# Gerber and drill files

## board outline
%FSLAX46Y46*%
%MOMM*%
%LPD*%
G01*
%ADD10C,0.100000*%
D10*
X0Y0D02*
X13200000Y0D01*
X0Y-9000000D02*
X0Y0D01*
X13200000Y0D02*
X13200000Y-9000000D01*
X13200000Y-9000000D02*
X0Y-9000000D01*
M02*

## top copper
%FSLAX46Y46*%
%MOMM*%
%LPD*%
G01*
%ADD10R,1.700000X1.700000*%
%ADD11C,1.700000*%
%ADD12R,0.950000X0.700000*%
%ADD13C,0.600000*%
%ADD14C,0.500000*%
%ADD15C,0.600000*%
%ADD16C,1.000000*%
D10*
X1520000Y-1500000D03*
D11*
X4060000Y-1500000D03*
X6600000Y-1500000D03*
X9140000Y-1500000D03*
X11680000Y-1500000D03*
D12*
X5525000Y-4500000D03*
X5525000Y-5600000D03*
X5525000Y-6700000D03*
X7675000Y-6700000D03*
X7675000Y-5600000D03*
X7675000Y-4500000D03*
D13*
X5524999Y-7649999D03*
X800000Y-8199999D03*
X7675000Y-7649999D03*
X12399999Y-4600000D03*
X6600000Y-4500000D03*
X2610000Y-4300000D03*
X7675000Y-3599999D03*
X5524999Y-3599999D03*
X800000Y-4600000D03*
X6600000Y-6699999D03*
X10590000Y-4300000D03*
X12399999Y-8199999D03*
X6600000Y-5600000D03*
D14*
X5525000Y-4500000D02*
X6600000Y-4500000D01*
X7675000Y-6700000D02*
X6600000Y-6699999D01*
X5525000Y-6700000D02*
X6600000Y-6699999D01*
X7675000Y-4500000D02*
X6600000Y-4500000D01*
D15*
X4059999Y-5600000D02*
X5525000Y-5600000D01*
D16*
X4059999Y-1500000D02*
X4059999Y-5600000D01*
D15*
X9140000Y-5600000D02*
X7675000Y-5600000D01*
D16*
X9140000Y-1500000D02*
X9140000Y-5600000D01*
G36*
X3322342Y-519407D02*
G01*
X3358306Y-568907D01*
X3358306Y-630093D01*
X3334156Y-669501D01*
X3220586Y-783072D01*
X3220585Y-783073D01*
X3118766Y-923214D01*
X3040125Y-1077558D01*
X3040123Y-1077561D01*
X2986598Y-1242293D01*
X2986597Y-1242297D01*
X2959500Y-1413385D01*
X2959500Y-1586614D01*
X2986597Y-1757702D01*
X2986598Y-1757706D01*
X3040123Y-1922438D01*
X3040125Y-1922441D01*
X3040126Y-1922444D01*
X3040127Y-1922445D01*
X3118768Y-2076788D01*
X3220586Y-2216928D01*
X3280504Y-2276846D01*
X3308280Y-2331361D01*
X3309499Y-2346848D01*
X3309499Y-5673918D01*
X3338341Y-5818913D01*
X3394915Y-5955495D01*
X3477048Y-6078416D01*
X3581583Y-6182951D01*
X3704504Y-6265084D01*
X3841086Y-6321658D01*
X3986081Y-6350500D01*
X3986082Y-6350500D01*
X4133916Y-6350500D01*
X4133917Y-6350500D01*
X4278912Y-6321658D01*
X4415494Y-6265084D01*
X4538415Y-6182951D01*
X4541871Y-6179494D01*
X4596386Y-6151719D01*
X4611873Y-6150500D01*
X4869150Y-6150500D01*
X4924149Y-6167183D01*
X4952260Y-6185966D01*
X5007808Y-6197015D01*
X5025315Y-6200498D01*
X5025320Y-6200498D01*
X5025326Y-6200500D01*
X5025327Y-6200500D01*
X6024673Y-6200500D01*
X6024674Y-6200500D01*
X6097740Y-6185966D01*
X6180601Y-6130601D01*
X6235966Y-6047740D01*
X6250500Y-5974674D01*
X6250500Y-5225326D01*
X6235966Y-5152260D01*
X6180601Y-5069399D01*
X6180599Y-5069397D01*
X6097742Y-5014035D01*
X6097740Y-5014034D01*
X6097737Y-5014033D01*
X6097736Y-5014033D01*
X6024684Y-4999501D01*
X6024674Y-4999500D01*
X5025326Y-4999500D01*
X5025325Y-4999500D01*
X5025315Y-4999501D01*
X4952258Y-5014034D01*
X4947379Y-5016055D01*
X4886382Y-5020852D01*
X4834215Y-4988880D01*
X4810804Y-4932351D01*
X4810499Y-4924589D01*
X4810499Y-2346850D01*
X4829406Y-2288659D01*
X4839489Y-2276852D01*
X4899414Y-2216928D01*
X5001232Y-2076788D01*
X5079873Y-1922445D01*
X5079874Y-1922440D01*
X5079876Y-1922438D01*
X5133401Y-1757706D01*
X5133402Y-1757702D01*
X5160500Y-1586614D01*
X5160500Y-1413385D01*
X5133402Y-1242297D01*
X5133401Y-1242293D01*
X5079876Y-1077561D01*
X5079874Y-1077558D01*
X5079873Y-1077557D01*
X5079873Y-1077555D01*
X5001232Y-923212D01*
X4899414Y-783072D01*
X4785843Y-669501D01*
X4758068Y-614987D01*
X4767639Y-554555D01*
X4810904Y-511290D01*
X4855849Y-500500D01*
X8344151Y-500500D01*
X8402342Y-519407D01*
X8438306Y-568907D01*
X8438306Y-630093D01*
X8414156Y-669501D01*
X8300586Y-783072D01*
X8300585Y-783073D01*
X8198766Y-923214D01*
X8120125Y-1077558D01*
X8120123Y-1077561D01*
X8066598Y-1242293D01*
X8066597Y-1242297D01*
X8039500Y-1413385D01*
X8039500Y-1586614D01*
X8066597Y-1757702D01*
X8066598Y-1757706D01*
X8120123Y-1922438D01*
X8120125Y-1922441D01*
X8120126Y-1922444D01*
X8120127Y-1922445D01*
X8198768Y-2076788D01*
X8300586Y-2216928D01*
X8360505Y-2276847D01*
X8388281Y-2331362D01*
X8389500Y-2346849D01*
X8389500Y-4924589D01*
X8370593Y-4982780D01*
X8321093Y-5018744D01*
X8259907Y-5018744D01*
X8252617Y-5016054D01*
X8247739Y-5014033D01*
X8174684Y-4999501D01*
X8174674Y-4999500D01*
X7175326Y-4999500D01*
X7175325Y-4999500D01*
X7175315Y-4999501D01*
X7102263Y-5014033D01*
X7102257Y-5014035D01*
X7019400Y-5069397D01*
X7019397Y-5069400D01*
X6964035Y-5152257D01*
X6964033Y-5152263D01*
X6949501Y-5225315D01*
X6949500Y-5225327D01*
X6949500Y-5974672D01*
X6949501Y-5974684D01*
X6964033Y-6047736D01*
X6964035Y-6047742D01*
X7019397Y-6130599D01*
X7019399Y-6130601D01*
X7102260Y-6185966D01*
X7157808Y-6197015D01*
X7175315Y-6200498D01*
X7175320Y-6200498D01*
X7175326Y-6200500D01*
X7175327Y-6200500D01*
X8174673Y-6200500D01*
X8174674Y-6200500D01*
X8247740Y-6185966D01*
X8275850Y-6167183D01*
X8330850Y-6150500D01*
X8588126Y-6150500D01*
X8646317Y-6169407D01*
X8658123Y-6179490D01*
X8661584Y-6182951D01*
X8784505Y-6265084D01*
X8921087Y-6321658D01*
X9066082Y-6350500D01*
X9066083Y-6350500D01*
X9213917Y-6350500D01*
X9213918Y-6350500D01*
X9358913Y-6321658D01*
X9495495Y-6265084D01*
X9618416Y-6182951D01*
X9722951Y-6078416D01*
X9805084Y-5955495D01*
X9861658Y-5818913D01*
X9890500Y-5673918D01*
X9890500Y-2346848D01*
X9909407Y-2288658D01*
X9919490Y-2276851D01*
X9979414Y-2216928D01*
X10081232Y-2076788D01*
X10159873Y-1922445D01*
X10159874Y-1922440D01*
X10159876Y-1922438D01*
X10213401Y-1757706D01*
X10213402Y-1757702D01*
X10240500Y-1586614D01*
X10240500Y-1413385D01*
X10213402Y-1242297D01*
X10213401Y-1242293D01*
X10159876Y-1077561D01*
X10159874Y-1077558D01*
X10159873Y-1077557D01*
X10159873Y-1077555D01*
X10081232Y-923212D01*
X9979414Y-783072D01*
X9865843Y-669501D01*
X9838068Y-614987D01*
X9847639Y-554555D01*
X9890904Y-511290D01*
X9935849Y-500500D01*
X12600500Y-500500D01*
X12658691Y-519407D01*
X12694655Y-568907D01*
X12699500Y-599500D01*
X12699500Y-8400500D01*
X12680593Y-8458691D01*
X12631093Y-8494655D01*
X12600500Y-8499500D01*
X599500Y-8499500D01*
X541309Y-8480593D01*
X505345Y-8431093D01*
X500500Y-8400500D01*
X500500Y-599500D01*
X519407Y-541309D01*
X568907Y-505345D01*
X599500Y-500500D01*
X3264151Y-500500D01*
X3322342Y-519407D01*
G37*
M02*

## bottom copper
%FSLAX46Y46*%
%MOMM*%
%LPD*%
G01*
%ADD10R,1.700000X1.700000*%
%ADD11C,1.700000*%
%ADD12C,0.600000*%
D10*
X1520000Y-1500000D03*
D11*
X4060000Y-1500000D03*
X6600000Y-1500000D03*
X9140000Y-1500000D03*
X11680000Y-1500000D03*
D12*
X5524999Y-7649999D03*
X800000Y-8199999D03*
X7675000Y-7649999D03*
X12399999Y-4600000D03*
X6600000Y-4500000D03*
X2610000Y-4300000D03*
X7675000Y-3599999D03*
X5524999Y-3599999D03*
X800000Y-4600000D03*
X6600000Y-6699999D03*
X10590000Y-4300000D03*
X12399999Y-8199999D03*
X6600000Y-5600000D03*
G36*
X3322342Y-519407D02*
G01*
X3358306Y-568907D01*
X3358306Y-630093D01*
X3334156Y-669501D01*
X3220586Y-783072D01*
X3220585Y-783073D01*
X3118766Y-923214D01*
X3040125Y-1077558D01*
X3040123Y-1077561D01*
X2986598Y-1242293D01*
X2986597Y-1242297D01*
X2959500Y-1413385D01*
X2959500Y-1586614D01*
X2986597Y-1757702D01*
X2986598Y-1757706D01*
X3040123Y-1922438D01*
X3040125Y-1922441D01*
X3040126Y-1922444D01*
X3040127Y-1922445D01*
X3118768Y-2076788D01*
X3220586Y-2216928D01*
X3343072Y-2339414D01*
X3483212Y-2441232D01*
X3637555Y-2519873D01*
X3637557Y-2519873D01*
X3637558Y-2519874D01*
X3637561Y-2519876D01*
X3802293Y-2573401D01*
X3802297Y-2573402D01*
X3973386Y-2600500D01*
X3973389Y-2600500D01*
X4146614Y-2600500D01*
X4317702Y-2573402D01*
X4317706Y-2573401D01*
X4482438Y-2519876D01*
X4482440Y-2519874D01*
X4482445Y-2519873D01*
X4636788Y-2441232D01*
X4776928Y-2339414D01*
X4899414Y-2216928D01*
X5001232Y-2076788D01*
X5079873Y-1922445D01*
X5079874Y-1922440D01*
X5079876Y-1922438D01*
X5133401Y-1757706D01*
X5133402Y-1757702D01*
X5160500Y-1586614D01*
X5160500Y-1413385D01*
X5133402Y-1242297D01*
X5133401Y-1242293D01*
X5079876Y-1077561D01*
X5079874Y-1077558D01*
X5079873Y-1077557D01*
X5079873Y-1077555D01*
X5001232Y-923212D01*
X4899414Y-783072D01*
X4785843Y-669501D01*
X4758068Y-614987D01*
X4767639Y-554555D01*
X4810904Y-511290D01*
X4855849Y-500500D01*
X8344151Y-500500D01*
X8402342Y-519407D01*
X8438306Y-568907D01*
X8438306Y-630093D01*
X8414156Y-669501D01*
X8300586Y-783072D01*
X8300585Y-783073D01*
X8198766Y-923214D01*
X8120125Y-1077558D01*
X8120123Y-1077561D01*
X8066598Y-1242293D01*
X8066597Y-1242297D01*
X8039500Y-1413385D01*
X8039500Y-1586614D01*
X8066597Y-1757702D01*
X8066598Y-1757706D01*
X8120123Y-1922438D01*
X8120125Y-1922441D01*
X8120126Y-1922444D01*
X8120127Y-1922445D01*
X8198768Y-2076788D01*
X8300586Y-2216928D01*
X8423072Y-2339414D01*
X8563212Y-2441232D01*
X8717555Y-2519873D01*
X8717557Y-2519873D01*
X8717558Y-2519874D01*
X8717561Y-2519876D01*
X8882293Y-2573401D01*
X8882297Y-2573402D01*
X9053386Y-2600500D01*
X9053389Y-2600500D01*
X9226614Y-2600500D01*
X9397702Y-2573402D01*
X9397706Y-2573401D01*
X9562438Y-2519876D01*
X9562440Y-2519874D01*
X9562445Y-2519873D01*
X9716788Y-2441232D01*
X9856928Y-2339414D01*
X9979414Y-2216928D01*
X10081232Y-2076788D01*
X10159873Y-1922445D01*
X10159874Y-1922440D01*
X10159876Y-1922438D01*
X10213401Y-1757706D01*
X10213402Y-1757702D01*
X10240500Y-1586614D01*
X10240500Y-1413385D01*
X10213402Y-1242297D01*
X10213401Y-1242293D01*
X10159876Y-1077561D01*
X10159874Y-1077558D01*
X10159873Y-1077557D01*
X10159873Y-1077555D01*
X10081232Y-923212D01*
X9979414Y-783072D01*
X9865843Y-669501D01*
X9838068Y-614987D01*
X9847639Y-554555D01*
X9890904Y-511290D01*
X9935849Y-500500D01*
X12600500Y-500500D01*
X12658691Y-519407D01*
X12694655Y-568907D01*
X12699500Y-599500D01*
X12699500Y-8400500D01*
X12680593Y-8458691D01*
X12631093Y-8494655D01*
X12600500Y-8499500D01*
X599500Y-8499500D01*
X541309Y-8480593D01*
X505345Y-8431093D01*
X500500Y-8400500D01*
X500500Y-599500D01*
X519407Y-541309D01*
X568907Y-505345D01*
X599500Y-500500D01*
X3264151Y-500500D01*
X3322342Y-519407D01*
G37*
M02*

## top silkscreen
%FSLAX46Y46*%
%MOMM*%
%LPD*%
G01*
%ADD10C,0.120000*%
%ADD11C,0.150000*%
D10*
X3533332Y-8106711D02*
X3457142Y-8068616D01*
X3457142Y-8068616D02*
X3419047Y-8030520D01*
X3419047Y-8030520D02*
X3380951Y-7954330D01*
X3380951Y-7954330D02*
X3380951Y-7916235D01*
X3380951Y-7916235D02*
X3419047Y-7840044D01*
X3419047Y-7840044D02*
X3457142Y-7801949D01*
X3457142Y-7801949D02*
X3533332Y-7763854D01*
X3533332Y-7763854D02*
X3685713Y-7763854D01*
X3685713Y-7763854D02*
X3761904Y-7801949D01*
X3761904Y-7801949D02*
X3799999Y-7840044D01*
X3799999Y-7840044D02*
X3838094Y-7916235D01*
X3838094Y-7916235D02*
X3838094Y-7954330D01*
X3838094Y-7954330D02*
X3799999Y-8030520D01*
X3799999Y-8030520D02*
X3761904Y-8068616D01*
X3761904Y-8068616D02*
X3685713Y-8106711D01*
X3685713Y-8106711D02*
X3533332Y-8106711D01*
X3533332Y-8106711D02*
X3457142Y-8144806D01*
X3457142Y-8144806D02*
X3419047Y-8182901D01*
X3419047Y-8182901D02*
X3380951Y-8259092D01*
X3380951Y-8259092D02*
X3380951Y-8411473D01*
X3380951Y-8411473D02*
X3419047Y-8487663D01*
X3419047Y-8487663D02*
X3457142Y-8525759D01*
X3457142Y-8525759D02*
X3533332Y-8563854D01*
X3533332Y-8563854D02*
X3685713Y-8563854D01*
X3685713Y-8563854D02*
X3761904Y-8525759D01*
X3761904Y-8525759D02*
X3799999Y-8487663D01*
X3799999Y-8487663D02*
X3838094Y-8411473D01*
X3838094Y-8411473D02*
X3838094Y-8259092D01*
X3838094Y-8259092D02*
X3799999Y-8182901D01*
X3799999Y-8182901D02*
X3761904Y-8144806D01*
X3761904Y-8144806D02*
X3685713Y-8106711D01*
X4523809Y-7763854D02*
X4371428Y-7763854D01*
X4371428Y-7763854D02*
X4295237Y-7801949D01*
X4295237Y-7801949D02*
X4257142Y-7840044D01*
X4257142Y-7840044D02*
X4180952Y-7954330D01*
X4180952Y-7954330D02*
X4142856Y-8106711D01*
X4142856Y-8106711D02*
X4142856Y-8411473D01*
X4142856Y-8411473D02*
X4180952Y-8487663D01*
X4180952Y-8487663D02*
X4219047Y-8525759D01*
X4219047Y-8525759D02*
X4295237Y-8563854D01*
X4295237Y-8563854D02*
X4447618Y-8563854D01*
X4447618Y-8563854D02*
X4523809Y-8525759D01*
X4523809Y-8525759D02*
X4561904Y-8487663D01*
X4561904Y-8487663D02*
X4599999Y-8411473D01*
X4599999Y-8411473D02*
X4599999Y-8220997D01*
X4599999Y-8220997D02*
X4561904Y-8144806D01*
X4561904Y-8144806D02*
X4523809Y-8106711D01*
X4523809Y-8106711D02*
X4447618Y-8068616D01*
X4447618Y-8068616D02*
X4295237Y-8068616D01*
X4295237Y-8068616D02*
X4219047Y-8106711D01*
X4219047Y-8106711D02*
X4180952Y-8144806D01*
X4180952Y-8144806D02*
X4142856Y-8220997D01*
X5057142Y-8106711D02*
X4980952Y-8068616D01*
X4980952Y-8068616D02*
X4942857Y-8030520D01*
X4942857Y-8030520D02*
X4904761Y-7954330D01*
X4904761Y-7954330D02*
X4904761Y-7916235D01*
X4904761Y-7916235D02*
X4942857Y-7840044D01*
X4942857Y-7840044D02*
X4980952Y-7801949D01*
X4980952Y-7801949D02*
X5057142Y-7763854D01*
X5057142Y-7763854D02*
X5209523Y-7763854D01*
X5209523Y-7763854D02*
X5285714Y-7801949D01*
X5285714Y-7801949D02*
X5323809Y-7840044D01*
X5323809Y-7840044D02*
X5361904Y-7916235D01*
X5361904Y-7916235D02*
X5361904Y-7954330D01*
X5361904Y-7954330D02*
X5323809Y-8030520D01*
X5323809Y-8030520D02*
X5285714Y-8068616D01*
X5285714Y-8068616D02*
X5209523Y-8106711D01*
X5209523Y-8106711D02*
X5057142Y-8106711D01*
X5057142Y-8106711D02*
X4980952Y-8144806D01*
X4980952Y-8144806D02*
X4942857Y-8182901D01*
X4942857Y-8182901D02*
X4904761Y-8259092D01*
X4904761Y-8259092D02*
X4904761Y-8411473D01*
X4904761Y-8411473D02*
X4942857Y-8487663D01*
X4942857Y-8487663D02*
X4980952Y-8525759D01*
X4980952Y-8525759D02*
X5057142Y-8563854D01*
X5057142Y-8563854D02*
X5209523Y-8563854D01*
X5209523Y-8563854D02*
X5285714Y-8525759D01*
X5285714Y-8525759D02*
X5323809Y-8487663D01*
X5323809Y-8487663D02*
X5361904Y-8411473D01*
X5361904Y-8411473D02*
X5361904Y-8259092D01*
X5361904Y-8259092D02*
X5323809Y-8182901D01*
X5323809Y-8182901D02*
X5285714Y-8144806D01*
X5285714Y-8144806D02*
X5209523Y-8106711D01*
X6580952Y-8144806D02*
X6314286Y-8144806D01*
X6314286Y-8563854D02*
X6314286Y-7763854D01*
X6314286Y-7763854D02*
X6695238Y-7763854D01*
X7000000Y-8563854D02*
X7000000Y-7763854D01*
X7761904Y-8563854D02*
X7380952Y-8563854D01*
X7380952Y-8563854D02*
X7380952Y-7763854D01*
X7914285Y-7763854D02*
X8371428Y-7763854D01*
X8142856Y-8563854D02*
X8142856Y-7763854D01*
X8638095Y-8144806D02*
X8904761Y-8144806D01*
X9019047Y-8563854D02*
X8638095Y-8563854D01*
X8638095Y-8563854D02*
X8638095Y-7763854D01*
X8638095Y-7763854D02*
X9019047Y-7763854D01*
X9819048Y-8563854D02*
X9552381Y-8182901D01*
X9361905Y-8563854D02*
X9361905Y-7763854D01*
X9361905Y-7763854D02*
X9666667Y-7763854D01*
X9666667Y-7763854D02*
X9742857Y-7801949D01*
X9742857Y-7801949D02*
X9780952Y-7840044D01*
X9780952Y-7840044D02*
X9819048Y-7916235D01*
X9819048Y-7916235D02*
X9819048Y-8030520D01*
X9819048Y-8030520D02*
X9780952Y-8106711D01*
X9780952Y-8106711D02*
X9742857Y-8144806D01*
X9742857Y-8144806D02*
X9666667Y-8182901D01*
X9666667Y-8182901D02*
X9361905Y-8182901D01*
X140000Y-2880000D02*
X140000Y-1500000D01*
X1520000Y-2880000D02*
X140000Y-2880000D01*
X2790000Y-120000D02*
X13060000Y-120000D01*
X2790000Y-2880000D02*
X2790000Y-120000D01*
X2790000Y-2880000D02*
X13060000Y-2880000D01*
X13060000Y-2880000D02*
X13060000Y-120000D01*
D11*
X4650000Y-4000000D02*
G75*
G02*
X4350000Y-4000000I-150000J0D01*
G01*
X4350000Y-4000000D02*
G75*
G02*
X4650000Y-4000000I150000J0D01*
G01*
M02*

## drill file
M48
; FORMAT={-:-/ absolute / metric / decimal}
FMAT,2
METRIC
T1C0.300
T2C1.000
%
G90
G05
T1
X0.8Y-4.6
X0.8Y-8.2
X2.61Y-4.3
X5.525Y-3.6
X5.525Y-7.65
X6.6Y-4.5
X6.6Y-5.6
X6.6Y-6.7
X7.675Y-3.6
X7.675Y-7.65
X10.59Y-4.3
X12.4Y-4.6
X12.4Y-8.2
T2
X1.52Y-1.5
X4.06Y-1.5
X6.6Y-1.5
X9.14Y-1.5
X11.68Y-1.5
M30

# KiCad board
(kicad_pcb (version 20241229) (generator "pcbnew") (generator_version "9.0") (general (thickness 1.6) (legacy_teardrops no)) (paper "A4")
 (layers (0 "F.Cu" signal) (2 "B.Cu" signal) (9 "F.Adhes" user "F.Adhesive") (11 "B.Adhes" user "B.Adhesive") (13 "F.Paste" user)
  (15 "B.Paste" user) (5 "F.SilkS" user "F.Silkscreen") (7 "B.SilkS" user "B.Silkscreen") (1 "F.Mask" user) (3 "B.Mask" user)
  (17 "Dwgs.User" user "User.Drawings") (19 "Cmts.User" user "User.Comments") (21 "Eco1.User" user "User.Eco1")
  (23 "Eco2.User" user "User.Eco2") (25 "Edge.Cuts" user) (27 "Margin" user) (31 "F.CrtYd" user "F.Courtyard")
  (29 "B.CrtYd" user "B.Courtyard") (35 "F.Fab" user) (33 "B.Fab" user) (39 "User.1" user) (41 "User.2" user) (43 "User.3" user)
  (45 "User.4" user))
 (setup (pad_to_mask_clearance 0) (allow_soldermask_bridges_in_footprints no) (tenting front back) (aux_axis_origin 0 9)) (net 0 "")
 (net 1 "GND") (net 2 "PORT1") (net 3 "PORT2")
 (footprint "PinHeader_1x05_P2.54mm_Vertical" (layer "F.Cu") (at 1.52 1.5 90)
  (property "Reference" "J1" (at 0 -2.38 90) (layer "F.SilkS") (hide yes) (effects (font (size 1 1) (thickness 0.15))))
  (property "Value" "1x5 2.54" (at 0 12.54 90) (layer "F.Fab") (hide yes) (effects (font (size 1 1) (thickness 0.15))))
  (fp_line (start -1.38 -1.38) (end 0 -1.38) (stroke (width 0.12) (type solid)) (layer "F.SilkS"))
  (fp_line (start -1.38 0) (end -1.38 -1.38) (stroke (width 0.12) (type solid)) (layer "F.SilkS"))
  (fp_line (start 1.38 1.27) (end 1.38 11.54) (stroke (width 0.12) (type solid)) (layer "F.SilkS"))
  (fp_line (start -1.38 1.27) (end 1.38 1.27) (stroke (width 0.12) (type solid)) (layer "F.SilkS"))
  (fp_line (start -1.38 1.27) (end -1.38 11.54) (stroke (width 0.12) (type solid)) (layer "F.SilkS"))
  (fp_line (start -1.38 11.54) (end 1.38 11.54) (stroke (width 0.12) (type solid)) (layer "F.SilkS"))
  (pad "1" thru_hole rect (at 0 0 90) (size 1.7 1.7) (drill 1) (layers "*.Cu" "*.Mask") (remove_unused_layers no) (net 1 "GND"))
  (pad "2" thru_hole circle (at 0 2.54 90) (size 1.7 1.7) (drill 1) (layers "*.Cu" "*.Mask") (remove_unused_layers no) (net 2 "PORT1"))
  (pad "3" thru_hole circle (at 0 5.08 90) (size 1.7 1.7) (drill 1) (layers "*.Cu" "*.Mask") (remove_unused_layers no) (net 1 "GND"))
  (pad "4" thru_hole circle (at 0 7.62 90) (size 1.7 1.7) (drill 1) (layers "*.Cu" "*.Mask") (remove_unused_layers no) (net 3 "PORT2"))
  (pad "5" thru_hole circle (at 0 10.16 90) (size 1.7 1.7) (drill 1) (layers "*.Cu" "*.Mask") (remove_unused_layers no) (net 1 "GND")))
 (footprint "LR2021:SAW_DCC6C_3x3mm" (layer "F.Cu") (at 6.6 5.6)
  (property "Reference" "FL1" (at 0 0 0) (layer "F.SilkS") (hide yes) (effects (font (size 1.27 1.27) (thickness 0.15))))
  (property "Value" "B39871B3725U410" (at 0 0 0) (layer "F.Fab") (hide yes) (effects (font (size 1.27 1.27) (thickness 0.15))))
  (fp_circle (center -2.1 -1.6) (end -1.95 -1.6) (stroke (width 0.15) (type default)) (fill no) (layer "F.SilkS"))
  (pad "1" smd rect (at -1.075 -1.1) (size 0.95 0.7) (layers "F.Cu" "F.Mask" "F.Paste") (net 1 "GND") (thermal_bridge_angle 45))
  (pad "2" smd rect (at -1.075 0) (size 0.95 0.7) (layers "F.Cu" "F.Mask" "F.Paste") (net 2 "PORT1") (thermal_bridge_angle 45))
  (pad "3" smd rect (at -1.075 1.1) (size 0.95 0.7) (layers "F.Cu" "F.Mask" "F.Paste") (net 1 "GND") (thermal_bridge_angle 45))
  (pad "4" smd rect (at 1.075 1.1) (size 0.95 0.7) (layers "F.Cu" "F.Mask" "F.Paste") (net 1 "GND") (thermal_bridge_angle 45))
  (pad "5" smd rect (at 1.075 0) (size 0.95 0.7) (layers "F.Cu" "F.Mask" "F.Paste") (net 3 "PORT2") (thermal_bridge_angle 45))
  (pad "6" smd rect (at 1.075 -1.1) (size 0.95 0.7) (layers "F.Cu" "F.Mask" "F.Paste") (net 1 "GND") (thermal_bridge_angle 45)))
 (gr_line (start 0 0) (end 13.2 0) (stroke (width 0.1) (type default)) (layer "Edge.Cuts"))
 (gr_line (start 0 9) (end 0 0) (stroke (width 0.1) (type default)) (layer "Edge.Cuts"))
 (gr_line (start 13.2 0) (end 13.2 9) (stroke (width 0.1) (type default)) (layer "Edge.Cuts"))
 (gr_line (start 13.2 9) (end 0 9) (stroke (width 0.1) (type default)) (layer "Edge.Cuts"))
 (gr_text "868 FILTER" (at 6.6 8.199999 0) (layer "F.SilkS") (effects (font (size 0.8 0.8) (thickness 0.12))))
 (segment (start 5.525 4.5) (end 6.6 4.5) (width 0.5) (layer "F.Cu") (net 1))
 (segment (start 7.675 6.7) (end 6.6 6.699999) (width 0.5) (layer "F.Cu") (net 1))
 (segment (start 5.525 6.7) (end 6.6 6.699999) (width 0.5) (layer "F.Cu") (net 1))
 (segment (start 7.675 4.5) (end 6.6 4.5) (width 0.5) (layer "F.Cu") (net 1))
 (via (at 5.524999 7.649999) (size 0.6) (drill 0.3) (layers "F.Cu" "B.Cu") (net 1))
 (via (at 0.8 8.199999) (size 0.6) (drill 0.3) (layers "F.Cu" "B.Cu") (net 1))
 (via (at 7.675 7.649999) (size 0.6) (drill 0.3) (layers "F.Cu" "B.Cu") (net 1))
 (via (at 12.399999 4.6) (size 0.6) (drill 0.3) (layers "F.Cu" "B.Cu") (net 1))
 (via (at 6.6 4.5) (size 0.6) (drill 0.3) (layers "F.Cu" "B.Cu") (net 1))
 (via (at 2.61 4.3) (size 0.6) (drill 0.3) (layers "F.Cu" "B.Cu") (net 1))
 (via (at 7.675 3.599999) (size 0.6) (drill 0.3) (layers "F.Cu" "B.Cu") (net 1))
 (via (at 5.524999 3.599999) (size 0.6) (drill 0.3) (layers "F.Cu" "B.Cu") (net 1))
 (via (at 0.8 4.6) (size 0.6) (drill 0.3) (layers "F.Cu" "B.Cu") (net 1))
 (via (at 6.6 6.699999) (size 0.6) (drill 0.3) (layers "F.Cu" "B.Cu") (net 1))
 (via (at 10.59 4.3) (size 0.6) (drill 0.3) (layers "F.Cu" "B.Cu") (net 1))
 (via (at 12.399999 8.199999) (size 0.6) (drill 0.3) (layers "F.Cu" "B.Cu") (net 1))
 (via (at 6.6 5.6) (size 0.6) (drill 0.3) (layers "F.Cu" "B.Cu") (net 1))
 (segment (start 4.059999 5.6) (end 5.525 5.6) (width 0.6) (layer "F.Cu") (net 2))
 (segment (start 4.059999 1.5) (end 4.059999 5.6) (width 1) (layer "F.Cu") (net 2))
 (segment (start 9.14 5.6) (end 7.675 5.6) (width 0.6) (layer "F.Cu") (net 3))
 (segment (start 9.14 1.5) (end 9.14 5.6) (width 1) (layer "F.Cu") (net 3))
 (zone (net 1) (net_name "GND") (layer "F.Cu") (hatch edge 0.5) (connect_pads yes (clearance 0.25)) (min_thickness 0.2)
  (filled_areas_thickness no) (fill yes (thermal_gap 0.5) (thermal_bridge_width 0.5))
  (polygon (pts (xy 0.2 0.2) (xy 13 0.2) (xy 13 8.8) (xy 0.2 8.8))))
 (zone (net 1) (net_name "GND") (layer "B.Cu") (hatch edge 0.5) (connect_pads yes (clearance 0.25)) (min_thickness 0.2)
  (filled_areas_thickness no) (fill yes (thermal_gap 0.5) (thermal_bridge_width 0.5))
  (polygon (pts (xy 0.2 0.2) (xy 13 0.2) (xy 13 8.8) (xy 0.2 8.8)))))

